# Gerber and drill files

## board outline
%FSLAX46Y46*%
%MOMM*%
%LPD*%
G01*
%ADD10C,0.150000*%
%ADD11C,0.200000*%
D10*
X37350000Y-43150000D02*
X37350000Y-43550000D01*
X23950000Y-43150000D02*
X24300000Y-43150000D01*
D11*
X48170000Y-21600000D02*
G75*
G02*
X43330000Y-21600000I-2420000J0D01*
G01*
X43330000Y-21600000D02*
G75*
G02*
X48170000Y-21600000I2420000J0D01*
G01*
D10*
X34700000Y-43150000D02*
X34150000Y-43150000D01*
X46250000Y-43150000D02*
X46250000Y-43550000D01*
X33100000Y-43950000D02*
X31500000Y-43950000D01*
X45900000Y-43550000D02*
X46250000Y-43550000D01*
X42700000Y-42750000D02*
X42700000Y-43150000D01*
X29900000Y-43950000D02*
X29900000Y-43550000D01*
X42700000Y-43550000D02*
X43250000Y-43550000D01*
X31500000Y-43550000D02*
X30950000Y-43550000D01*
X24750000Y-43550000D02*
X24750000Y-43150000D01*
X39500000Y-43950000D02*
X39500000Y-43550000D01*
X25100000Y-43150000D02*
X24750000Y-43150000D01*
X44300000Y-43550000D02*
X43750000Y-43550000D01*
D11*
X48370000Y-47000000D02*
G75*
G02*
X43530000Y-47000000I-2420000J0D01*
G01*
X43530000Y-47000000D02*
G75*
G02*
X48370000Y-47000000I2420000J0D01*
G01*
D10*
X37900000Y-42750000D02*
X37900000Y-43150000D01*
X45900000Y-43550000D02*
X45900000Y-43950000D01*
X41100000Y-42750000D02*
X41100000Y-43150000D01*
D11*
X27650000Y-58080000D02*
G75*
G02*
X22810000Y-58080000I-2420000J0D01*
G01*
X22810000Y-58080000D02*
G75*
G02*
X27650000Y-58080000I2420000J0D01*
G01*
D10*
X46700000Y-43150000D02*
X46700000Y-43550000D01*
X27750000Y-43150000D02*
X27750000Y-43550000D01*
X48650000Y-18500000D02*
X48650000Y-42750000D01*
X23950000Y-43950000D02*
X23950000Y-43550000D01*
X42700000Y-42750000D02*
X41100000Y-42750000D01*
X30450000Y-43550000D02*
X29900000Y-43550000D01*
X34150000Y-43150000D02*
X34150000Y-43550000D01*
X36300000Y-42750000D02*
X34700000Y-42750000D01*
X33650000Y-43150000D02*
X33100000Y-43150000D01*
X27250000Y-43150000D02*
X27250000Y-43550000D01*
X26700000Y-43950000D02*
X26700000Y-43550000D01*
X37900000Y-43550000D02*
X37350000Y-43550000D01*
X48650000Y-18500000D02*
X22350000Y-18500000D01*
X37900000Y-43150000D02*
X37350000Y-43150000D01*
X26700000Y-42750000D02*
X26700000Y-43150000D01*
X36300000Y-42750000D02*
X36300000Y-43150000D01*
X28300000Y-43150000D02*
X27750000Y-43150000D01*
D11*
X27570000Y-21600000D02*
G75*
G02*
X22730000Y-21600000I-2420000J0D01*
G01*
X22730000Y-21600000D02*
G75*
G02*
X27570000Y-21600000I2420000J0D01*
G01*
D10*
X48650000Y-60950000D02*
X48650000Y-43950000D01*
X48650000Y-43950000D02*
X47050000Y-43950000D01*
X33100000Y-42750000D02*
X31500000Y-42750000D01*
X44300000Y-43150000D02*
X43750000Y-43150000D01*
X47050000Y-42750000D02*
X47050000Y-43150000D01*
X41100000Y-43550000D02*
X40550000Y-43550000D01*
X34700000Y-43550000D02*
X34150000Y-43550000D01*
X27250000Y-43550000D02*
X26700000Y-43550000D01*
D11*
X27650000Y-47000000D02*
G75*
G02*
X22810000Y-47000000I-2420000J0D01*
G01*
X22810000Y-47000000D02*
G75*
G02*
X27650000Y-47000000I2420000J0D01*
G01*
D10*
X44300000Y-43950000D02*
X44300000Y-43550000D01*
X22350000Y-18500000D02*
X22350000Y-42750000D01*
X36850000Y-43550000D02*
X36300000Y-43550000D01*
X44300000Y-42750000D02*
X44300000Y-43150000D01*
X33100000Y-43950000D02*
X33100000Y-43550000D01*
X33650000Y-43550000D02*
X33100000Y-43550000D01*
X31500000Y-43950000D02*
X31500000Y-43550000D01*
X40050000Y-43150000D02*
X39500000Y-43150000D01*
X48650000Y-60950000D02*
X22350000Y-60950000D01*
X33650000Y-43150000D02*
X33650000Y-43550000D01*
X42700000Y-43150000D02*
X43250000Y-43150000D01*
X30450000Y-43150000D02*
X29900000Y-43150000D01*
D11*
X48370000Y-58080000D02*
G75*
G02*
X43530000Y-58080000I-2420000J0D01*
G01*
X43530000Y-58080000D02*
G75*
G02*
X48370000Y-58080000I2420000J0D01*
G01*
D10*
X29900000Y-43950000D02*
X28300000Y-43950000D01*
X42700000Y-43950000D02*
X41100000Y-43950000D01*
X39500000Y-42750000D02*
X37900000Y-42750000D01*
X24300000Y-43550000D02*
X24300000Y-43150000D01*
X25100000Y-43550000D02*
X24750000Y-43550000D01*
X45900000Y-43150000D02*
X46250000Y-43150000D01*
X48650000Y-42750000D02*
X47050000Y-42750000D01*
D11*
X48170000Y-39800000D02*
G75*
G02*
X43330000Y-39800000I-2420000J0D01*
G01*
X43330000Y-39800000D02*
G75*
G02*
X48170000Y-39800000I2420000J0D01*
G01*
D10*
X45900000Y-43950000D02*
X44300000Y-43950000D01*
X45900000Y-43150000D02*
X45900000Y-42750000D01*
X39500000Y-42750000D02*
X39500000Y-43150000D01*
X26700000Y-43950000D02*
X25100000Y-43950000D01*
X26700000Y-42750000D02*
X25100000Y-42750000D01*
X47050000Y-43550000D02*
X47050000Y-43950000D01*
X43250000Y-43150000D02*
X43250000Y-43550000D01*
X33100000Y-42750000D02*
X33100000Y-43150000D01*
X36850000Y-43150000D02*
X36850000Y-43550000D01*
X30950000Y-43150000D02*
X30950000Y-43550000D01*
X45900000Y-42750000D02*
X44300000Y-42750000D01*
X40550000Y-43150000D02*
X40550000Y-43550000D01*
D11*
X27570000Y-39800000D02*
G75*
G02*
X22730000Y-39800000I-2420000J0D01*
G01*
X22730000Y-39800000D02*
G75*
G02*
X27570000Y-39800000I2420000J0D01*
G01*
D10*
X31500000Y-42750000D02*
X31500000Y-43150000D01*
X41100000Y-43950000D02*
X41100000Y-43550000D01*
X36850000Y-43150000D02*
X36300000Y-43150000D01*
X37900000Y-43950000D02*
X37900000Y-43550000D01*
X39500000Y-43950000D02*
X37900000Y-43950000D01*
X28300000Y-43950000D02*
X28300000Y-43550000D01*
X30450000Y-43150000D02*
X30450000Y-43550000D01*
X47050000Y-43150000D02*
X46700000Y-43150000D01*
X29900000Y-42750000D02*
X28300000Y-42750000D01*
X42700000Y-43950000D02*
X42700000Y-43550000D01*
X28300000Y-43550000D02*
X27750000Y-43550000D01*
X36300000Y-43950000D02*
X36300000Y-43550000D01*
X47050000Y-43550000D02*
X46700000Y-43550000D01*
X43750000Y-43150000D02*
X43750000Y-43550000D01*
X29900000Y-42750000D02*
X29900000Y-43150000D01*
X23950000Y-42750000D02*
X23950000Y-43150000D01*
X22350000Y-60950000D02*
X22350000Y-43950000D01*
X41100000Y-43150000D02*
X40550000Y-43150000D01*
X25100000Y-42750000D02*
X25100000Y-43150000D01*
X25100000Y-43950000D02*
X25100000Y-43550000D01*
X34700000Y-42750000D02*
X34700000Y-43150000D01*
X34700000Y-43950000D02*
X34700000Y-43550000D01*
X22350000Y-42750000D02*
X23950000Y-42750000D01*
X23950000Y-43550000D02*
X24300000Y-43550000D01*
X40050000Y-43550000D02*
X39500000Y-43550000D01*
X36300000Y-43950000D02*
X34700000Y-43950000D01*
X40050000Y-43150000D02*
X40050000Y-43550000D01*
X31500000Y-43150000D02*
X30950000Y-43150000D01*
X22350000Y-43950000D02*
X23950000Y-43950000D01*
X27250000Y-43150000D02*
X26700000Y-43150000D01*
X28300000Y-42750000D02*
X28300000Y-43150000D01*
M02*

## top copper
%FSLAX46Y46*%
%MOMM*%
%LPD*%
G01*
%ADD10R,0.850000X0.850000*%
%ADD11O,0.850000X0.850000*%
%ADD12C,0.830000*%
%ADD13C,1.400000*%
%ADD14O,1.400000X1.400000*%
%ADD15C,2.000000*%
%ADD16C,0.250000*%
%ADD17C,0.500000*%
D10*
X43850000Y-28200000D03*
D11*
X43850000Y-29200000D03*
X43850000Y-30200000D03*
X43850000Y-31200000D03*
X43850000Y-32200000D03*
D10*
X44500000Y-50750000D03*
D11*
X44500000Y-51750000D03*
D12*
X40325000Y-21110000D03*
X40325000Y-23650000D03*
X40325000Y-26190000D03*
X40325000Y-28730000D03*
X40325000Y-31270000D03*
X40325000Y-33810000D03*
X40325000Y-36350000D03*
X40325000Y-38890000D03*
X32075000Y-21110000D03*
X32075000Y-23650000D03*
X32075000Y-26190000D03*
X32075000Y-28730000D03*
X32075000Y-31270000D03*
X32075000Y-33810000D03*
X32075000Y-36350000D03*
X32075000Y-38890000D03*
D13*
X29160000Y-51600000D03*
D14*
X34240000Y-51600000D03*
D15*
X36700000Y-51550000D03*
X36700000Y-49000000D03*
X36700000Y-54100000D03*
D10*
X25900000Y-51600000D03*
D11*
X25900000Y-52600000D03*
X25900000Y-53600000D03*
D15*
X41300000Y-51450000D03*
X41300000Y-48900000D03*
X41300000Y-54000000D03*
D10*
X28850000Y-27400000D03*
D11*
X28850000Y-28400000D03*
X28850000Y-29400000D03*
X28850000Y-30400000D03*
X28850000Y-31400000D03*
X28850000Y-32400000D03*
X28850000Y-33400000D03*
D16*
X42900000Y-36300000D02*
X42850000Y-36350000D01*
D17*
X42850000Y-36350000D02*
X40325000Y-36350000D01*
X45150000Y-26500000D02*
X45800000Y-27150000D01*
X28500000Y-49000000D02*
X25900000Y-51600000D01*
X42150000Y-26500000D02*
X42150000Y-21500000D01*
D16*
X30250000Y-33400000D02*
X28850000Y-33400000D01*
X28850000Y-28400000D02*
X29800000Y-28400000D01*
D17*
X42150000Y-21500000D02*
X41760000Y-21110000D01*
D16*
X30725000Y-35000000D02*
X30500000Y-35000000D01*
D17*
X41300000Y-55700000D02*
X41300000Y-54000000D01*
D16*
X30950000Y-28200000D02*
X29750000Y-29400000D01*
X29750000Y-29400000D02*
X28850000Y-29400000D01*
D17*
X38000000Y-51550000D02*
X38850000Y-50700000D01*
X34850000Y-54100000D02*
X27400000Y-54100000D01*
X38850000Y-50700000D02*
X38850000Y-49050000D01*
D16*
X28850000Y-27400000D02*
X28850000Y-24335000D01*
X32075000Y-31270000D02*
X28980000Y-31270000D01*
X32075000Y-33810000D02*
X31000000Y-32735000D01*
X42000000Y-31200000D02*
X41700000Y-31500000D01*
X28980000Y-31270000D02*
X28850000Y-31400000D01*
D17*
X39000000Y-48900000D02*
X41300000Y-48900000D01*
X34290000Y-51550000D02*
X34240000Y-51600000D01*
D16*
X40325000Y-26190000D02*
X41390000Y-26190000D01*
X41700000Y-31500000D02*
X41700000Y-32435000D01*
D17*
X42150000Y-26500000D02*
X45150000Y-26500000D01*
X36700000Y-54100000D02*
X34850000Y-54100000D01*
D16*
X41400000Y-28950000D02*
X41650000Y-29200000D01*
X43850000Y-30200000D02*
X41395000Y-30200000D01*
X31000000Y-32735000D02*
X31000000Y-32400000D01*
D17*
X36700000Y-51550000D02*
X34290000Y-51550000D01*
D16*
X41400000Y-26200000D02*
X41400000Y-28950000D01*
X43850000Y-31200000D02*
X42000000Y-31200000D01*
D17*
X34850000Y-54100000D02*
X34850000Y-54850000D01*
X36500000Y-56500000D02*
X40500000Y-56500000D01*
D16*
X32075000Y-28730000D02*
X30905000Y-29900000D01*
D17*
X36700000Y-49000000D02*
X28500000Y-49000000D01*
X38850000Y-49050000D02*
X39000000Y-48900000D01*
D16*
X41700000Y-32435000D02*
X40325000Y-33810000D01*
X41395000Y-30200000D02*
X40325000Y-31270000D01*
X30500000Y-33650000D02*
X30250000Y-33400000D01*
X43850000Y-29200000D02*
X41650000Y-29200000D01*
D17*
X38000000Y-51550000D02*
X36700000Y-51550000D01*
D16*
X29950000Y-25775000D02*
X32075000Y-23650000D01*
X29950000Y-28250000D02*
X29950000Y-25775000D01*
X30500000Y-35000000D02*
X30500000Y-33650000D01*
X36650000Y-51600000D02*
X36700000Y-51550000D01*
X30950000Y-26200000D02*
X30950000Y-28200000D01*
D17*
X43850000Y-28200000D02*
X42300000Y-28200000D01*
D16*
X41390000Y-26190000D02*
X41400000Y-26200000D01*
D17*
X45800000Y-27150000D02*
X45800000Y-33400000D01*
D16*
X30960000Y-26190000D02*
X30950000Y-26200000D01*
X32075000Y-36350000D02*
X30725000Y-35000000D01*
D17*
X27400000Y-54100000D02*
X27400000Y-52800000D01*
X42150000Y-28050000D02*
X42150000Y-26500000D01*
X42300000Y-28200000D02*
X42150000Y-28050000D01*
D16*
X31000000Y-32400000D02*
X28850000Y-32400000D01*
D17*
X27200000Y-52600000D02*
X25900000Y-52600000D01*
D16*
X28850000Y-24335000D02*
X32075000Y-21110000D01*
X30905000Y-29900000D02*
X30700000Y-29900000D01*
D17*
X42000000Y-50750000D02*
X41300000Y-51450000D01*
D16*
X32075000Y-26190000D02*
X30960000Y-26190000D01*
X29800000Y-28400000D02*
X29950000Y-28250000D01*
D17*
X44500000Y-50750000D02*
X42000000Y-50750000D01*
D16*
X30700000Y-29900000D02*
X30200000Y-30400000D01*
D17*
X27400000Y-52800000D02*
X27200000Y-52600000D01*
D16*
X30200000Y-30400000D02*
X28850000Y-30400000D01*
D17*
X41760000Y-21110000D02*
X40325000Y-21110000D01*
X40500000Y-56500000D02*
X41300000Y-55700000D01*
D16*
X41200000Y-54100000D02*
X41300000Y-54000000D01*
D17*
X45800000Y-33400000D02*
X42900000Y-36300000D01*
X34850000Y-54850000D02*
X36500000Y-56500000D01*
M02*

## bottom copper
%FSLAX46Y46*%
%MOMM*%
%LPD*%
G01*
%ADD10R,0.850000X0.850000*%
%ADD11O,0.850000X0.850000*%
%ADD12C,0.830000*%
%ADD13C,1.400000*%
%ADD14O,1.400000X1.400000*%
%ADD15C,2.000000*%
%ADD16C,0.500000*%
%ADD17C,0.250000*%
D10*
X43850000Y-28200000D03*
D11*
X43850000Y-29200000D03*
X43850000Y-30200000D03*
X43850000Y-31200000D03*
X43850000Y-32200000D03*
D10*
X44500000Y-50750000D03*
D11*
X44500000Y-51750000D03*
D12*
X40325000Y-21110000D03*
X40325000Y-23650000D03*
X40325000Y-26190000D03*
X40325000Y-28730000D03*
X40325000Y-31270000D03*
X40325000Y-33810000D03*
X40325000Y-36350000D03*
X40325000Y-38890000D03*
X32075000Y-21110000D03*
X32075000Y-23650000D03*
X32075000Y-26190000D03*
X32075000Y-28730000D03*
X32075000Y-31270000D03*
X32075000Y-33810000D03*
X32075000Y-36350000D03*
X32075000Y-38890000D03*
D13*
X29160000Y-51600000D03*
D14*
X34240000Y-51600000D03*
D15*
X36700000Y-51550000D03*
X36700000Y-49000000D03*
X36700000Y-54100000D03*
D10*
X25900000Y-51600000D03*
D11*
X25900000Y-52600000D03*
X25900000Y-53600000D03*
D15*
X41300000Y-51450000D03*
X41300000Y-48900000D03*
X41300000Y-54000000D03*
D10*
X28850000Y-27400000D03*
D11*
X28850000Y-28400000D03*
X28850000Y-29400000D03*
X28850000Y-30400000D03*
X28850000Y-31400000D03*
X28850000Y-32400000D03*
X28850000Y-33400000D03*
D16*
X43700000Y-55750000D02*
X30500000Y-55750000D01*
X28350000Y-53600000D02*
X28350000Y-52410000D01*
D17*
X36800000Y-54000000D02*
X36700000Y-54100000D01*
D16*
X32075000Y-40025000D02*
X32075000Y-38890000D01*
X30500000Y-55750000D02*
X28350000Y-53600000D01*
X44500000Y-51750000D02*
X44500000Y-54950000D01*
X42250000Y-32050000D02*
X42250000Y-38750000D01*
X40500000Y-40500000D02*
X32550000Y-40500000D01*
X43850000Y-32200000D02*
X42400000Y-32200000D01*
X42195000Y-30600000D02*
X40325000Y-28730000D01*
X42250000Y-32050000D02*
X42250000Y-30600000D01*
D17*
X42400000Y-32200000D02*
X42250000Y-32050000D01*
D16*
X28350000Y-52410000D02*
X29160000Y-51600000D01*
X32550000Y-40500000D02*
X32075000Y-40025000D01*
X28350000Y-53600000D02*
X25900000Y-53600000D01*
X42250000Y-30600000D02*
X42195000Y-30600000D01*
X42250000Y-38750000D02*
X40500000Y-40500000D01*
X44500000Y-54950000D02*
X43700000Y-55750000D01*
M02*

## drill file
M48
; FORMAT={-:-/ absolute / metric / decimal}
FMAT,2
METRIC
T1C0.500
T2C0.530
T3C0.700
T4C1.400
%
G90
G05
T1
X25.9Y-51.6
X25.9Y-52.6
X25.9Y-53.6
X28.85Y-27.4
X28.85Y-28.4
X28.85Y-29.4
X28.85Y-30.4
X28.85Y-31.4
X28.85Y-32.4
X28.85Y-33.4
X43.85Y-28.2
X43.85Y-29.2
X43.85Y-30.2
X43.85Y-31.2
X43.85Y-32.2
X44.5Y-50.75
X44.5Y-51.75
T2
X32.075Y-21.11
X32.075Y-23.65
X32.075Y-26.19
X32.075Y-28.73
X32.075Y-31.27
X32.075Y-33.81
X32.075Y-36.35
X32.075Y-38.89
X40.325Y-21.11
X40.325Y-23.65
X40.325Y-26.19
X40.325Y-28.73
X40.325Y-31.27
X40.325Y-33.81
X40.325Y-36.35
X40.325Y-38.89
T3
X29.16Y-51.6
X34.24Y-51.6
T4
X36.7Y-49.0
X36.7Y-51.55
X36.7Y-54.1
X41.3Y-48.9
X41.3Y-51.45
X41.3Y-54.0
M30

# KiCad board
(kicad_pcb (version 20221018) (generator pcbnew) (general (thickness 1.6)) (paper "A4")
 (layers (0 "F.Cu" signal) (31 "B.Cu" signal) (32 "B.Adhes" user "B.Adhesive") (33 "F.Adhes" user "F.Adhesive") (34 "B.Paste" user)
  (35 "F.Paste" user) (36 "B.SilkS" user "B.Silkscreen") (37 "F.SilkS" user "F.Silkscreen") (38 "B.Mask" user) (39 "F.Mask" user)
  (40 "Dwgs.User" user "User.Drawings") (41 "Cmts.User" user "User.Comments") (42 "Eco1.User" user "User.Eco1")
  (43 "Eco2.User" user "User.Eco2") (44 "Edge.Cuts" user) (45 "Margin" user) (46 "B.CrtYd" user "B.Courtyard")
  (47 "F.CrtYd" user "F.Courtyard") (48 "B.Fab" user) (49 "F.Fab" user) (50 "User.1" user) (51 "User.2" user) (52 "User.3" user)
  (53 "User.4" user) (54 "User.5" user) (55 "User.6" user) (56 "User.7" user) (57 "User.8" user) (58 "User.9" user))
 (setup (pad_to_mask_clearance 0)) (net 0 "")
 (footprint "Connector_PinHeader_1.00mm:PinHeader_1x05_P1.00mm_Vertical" (layer "F.Cu") (at 43.85 28.2)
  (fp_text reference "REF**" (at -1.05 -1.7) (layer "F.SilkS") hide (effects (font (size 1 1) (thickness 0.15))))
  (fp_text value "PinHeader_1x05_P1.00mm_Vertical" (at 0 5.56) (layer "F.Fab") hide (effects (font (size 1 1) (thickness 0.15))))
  (pad "1" thru_hole rect (at 0 0) (size 0.85 0.85) (drill 0.5) (layers "*.Cu" "*.Mask"))
  (pad "2" thru_hole oval (at 0 1) (size 0.85 0.85) (drill 0.5) (layers "*.Cu" "*.Mask"))
  (pad "3" thru_hole oval (at 0 2) (size 0.85 0.85) (drill 0.5) (layers "*.Cu" "*.Mask"))
  (pad "4" thru_hole oval (at 0 3) (size 0.85 0.85) (drill 0.5) (layers "*.Cu" "*.Mask"))
  (pad "5" thru_hole oval (at 0 4) (size 0.85 0.85) (drill 0.5) (layers "*.Cu" "*.Mask")))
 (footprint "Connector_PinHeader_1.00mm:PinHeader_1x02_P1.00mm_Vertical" (layer "F.Cu") (at 44.5 50.75)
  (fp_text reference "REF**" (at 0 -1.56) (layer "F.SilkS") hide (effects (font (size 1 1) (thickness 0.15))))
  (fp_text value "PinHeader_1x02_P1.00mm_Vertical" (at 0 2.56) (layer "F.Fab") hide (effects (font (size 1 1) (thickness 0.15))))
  (pad "1" thru_hole rect (at 0 0) (size 0.85 0.85) (drill 0.5) (layers "*.Cu" "*.Mask"))
  (pad "2" thru_hole oval (at 0 1) (size 0.85 0.85) (drill 0.5) (layers "*.Cu" "*.Mask")))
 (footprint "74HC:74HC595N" (layer "F.Cu") (at 36.2 30 -90)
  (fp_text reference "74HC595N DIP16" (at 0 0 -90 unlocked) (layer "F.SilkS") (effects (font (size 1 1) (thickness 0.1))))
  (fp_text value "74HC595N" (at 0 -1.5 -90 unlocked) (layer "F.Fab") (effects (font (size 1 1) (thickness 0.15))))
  (pad "1" thru_hole circle (at -8.89 -4.125 270) (size 0.83 0.83) (drill 0.53) (layers "*.Cu" "*.Mask"))
  (pad "2" thru_hole circle (at -6.35 -4.125 270) (size 0.83 0.83) (drill 0.53) (layers "*.Cu" "*.Mask"))
  (pad "3" thru_hole circle (at -3.81 -4.125 270) (size 0.83 0.83) (drill 0.53) (layers "*.Cu" "*.Mask"))
  (pad "4" thru_hole circle (at -1.27 -4.125 270) (size 0.83 0.83) (drill 0.53) (layers "*.Cu" "*.Mask"))
  (pad "5" thru_hole circle (at 1.27 -4.125 270) (size 0.83 0.83) (drill 0.53) (layers "*.Cu" "*.Mask"))
  (pad "6" thru_hole circle (at 3.81 -4.125 270) (size 0.83 0.83) (drill 0.53) (layers "*.Cu" "*.Mask"))
  (pad "7" thru_hole circle (at 6.35 -4.125 270) (size 0.83 0.83) (drill 0.53) (layers "*.Cu" "*.Mask"))
  (pad "8" thru_hole circle (at 8.89 -4.125 270) (size 0.83 0.83) (drill 0.53) (layers "*.Cu" "*.Mask"))
  (pad "9" thru_hole circle (at -8.89 4.125 270) (size 0.83 0.83) (drill 0.53) (layers "*.Cu" "*.Mask"))
  (pad "10" thru_hole circle (at -6.35 4.125 270) (size 0.83 0.83) (drill 0.53) (layers "*.Cu" "*.Mask"))
  (pad "11" thru_hole circle (at -3.81 4.125 270) (size 0.83 0.83) (drill 0.53) (layers "*.Cu" "*.Mask"))
  (pad "12" thru_hole circle (at -1.27 4.125 270) (size 0.83 0.83) (drill 0.53) (layers "*.Cu" "*.Mask"))
  (pad "13" thru_hole circle (at 1.27 4.125 270) (size 0.83 0.83) (drill 0.53) (layers "*.Cu" "*.Mask"))
  (pad "14" thru_hole circle (at 3.81 4.125 270) (size 0.83 0.83) (drill 0.53) (layers "*.Cu" "*.Mask"))
  (pad "15" thru_hole circle (at 6.35 4.125 270) (size 0.83 0.83) (drill 0.53) (layers "*.Cu" "*.Mask"))
  (pad "16" thru_hole circle (at 8.89 4.125 270) (size 0.83 0.83) (drill 0.53) (layers "*.Cu" "*.Mask")))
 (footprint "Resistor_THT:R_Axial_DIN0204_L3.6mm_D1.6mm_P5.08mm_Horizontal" (layer "F.Cu") (at 29.16 51.6)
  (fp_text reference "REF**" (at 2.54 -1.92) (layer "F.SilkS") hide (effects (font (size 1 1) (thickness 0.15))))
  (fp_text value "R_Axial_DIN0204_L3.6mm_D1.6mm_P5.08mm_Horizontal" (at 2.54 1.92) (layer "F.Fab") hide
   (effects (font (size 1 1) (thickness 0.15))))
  (pad "1" thru_hole circle (at 0 0) (size 1.4 1.4) (drill 0.7) (layers "*.Cu" "*.Mask"))
  (pad "2" thru_hole oval (at 5.08 0) (size 1.4 1.4) (drill 0.7) (layers "*.Cu" "*.Mask")))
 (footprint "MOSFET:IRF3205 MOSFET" (layer "F.Cu") (at 36.7 51.55)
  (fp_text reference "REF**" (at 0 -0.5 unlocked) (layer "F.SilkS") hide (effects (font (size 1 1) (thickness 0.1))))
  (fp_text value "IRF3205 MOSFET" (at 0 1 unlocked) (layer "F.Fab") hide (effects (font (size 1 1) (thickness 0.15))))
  (pad "D" thru_hole circle (at 0 0) (size 2 2) (drill 1.4) (layers "*.Cu" "*.Mask"))
  (pad "G" thru_hole circle (at 0 -2.55) (size 2 2) (drill 1.4) (layers "*.Cu" "*.Mask"))
  (pad "S" thru_hole circle (at 0 2.55) (size 2 2) (drill 1.4) (layers "*.Cu" "*.Mask")))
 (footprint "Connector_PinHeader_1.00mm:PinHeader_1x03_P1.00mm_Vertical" (layer "F.Cu") (at 25.9 51.6)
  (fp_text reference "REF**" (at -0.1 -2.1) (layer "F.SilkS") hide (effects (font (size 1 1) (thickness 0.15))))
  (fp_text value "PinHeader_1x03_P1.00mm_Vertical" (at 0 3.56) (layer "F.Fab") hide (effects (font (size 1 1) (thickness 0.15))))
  (pad "1" thru_hole rect (at 0 0) (size 0.85 0.85) (drill 0.5) (layers "*.Cu" "*.Mask"))
  (pad "2" thru_hole oval (at 0 1) (size 0.85 0.85) (drill 0.5) (layers "*.Cu" "*.Mask"))
  (pad "3" thru_hole oval (at 0 2) (size 0.85 0.85) (drill 0.5) (layers "*.Cu" "*.Mask")))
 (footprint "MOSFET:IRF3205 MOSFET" (layer "F.Cu") (at 41.3 51.45)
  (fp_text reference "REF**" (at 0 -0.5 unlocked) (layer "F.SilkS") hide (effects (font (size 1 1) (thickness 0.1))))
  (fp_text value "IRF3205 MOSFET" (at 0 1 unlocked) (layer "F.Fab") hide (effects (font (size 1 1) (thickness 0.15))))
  (pad "D" thru_hole circle (at 0 0) (size 2 2) (drill 1.4) (layers "*.Cu" "*.Mask"))
  (pad "G" thru_hole circle (at 0 -2.55) (size 2 2) (drill 1.4) (layers "*.Cu" "*.Mask"))
  (pad "S" thru_hole circle (at 0 2.55) (size 2 2) (drill 1.4) (layers "*.Cu" "*.Mask")))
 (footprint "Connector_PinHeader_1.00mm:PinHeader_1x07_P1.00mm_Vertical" (layer "F.Cu") (at 28.85 27.4)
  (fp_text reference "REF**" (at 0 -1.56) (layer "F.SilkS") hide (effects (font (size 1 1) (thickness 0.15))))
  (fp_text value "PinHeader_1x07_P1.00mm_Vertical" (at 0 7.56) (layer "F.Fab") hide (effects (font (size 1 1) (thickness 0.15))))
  (pad "1" thru_hole rect (at 0 0) (size 0.85 0.85) (drill 0.5) (layers "*.Cu" "*.Mask"))
  (pad "2" thru_hole oval (at 0 1) (size 0.85 0.85) (drill 0.5) (layers "*.Cu" "*.Mask"))
  (pad "3" thru_hole oval (at 0 2) (size 0.85 0.85) (drill 0.5) (layers "*.Cu" "*.Mask"))
  (pad "4" thru_hole oval (at 0 3) (size 0.85 0.85) (drill 0.5) (layers "*.Cu" "*.Mask"))
  (pad "5" thru_hole oval (at 0 4) (size 0.85 0.85) (drill 0.5) (layers "*.Cu" "*.Mask"))
  (pad "6" thru_hole oval (at 0 5) (size 0.85 0.85) (drill 0.5) (layers "*.Cu" "*.Mask"))
  (pad "7" thru_hole oval (at 0 6) (size 0.85 0.85) (drill 0.5) (layers "*.Cu" "*.Mask")))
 (gr_line (start 37.35 43.15) (end 37.35 43.55) (stroke (width 0.15) (type default)) (layer "Edge.Cuts"))
 (gr_line (start 23.95 43.15) (end 24.3 43.15) (stroke (width 0.15) (type default)) (layer "Edge.Cuts"))
 (gr_circle (center 45.75 21.6) (end 48.17 21.6) (stroke (width 0.2) (type default)) (fill none) (layer "Edge.Cuts"))
 (gr_line (start 34.7 43.15) (end 34.15 43.15) (stroke (width 0.15) (type default)) (layer "Edge.Cuts"))
 (gr_line (start 46.25 43.15) (end 46.25 43.55) (stroke (width 0.15) (type default)) (layer "Edge.Cuts"))
 (gr_line (start 33.1 43.95) (end 31.5 43.95) (stroke (width 0.15) (type default)) (layer "Edge.Cuts"))
 (gr_line (start 45.9 43.55) (end 46.25 43.55) (stroke (width 0.15) (type default)) (layer "Edge.Cuts"))
 (gr_line (start 42.7 42.75) (end 42.7 43.15) (stroke (width 0.15) (type default)) (layer "Edge.Cuts"))
 (gr_line (start 29.9 43.95) (end 29.9 43.55) (stroke (width 0.15) (type default)) (layer "Edge.Cuts"))
 (gr_line (start 42.7 43.55) (end 43.25 43.55) (stroke (width 0.15) (type default)) (layer "Edge.Cuts"))
 (gr_line (start 31.5 43.55) (end 30.95 43.55) (stroke (width 0.15) (type default)) (layer "Edge.Cuts"))
 (gr_line (start 24.75 43.55) (end 24.75 43.15) (stroke (width 0.15) (type default)) (layer "Edge.Cuts"))
 (gr_line (start 39.5 43.95) (end 39.5 43.55) (stroke (width 0.15) (type default)) (layer "Edge.Cuts"))
 (gr_line (start 25.1 43.15) (end 24.75 43.15) (stroke (width 0.15) (type default)) (layer "Edge.Cuts"))
 (gr_line (start 44.3 43.55) (end 43.75 43.55) (stroke (width 0.15) (type default)) (layer "Edge.Cuts"))
 (gr_circle (center 45.95 47) (end 48.37 47) (stroke (width 0.2) (type default)) (fill none) (layer "Edge.Cuts"))
 (gr_line (start 37.9 42.75) (end 37.9 43.15) (stroke (width 0.15) (type default)) (layer "Edge.Cuts"))
 (gr_line (start 45.9 43.55) (end 45.9 43.95) (stroke (width 0.15) (type default)) (layer "Edge.Cuts"))
 (gr_line (start 41.1 42.75) (end 41.1 43.15) (stroke (width 0.15) (type default)) (layer "Edge.Cuts"))
 (gr_circle (center 25.23 58.08) (end 27.65 58.08) (stroke (width 0.2) (type default)) (fill none) (layer "Edge.Cuts"))
 (gr_line (start 46.7 43.15) (end 46.7 43.55) (stroke (width 0.15) (type default)) (layer "Edge.Cuts"))
 (gr_line (start 27.75 43.15) (end 27.75 43.55) (stroke (width 0.15) (type default)) (layer "Edge.Cuts"))
 (gr_line (start 48.65 18.5) (end 48.65 42.75) (stroke (width 0.15) (type default)) (layer "Edge.Cuts"))
 (gr_line (start 23.95 43.95) (end 23.95 43.55) (stroke (width 0.15) (type default)) (layer "Edge.Cuts"))
 (gr_line (start 42.7 42.75) (end 41.1 42.75) (stroke (width 0.15) (type default)) (layer "Edge.Cuts"))
 (gr_line (start 30.45 43.55) (end 29.9 43.55) (stroke (width 0.15) (type default)) (layer "Edge.Cuts"))
 (gr_line (start 34.15 43.15) (end 34.15 43.55) (stroke (width 0.15) (type default)) (layer "Edge.Cuts"))
 (gr_line (start 36.3 42.75) (end 34.7 42.75) (stroke (width 0.15) (type default)) (layer "Edge.Cuts"))
 (gr_line (start 33.65 43.15) (end 33.1 43.15) (stroke (width 0.15) (type default)) (layer "Edge.Cuts"))
 (gr_line (start 27.25 43.15) (end 27.25 43.55) (stroke (width 0.15) (type default)) (layer "Edge.Cuts"))
 (gr_line (start 26.7 43.95) (end 26.7 43.55) (stroke (width 0.15) (type default)) (layer "Edge.Cuts"))
 (gr_line (start 37.9 43.55) (end 37.35 43.55) (stroke (width 0.15) (type default)) (layer "Edge.Cuts"))
 (gr_line (start 48.65 18.5) (end 22.35 18.5) (stroke (width 0.15) (type default)) (layer "Edge.Cuts"))
 (gr_line (start 37.9 43.15) (end 37.35 43.15) (stroke (width 0.15) (type default)) (layer "Edge.Cuts"))
 (gr_line (start 26.7 42.75) (end 26.7 43.15) (stroke (width 0.15) (type default)) (layer "Edge.Cuts"))
 (gr_line (start 36.3 42.75) (end 36.3 43.15) (stroke (width 0.15) (type default)) (layer "Edge.Cuts"))
 (gr_line (start 28.3 43.15) (end 27.75 43.15) (stroke (width 0.15) (type default)) (layer "Edge.Cuts"))
 (gr_circle (center 25.15 21.6) (end 27.57 21.6) (stroke (width 0.2) (type default)) (fill none) (layer "Edge.Cuts"))
 (gr_line (start 48.65 60.95) (end 48.65 43.95) (stroke (width 0.15) (type default)) (layer "Edge.Cuts"))
 (gr_line (start 48.65 43.95) (end 47.05 43.95) (stroke (width 0.15) (type default)) (layer "Edge.Cuts"))
 (gr_line (start 33.1 42.75) (end 31.5 42.75) (stroke (width 0.15) (type default)) (layer "Edge.Cuts"))
 (gr_line (start 44.3 43.15) (end 43.75 43.15) (stroke (width 0.15) (type default)) (layer "Edge.Cuts"))
 (gr_line (start 47.05 42.75) (end 47.05 43.15) (stroke (width 0.15) (type default)) (layer "Edge.Cuts"))
 (gr_line (start 41.1 43.55) (end 40.55 43.55) (stroke (width 0.15) (type default)) (layer "Edge.Cuts"))
 (gr_line (start 34.7 43.55) (end 34.15 43.55) (stroke (width 0.15) (type default)) (layer "Edge.Cuts"))
 (gr_line (start 27.25 43.55) (end 26.7 43.55) (stroke (width 0.15) (type default)) (layer "Edge.Cuts"))
 (gr_circle (center 25.23 47) (end 27.65 47) (stroke (width 0.2) (type default)) (fill none) (layer "Edge.Cuts"))
 (gr_line (start 44.3 43.95) (end 44.3 43.55) (stroke (width 0.15) (type default)) (layer "Edge.Cuts"))
 (gr_line (start 22.35 18.5) (end 22.35 42.75) (stroke (width 0.15) (type default)) (layer "Edge.Cuts"))
 (gr_line (start 36.85 43.55) (end 36.3 43.55) (stroke (width 0.15) (type default)) (layer "Edge.Cuts"))
 (gr_line (start 44.3 42.75) (end 44.3 43.15) (stroke (width 0.15) (type default)) (layer "Edge.Cuts"))
 (gr_line (start 33.1 43.95) (end 33.1 43.55) (stroke (width 0.15) (type default)) (layer "Edge.Cuts"))
 (gr_line (start 33.65 43.55) (end 33.1 43.55) (stroke (width 0.15) (type default)) (layer "Edge.Cuts"))
 (gr_line (start 31.5 43.95) (end 31.5 43.55) (stroke (width 0.15) (type default)) (layer "Edge.Cuts"))
 (gr_line (start 40.05 43.15) (end 39.5 43.15) (stroke (width 0.15) (type default)) (layer "Edge.Cuts"))
 (gr_line (start 48.65 60.95) (end 22.35 60.95) (stroke (width 0.15) (type default)) (layer "Edge.Cuts"))
 (gr_line (start 33.65 43.15) (end 33.65 43.55) (stroke (width 0.15) (type default)) (layer "Edge.Cuts"))
 (gr_line (start 42.7 43.15) (end 43.25 43.15) (stroke (width 0.15) (type default)) (layer "Edge.Cuts"))
 (gr_line (start 30.45 43.15) (end 29.9 43.15) (stroke (width 0.15) (type default)) (layer "Edge.Cuts"))
 (gr_circle (center 45.95 58.08) (end 48.37 58.08) (stroke (width 0.2) (type default)) (fill none) (layer "Edge.Cuts"))
 (gr_line (start 29.9 43.95) (end 28.3 43.95) (stroke (width 0.15) (type default)) (layer "Edge.Cuts"))
 (gr_line (start 42.7 43.95) (end 41.1 43.95) (stroke (width 0.15) (type default)) (layer "Edge.Cuts"))
 (gr_line (start 39.5 42.75) (end 37.9 42.75) (stroke (width 0.15) (type default)) (layer "Edge.Cuts"))
 (gr_line (start 24.3 43.55) (end 24.3 43.15) (stroke (width 0.15) (type default)) (layer "Edge.Cuts"))
 (gr_line (start 25.1 43.55) (end 24.75 43.55) (stroke (width 0.15) (type default)) (layer "Edge.Cuts"))
 (gr_line (start 45.9 43.15) (end 46.25 43.15) (stroke (width 0.15) (type default)) (layer "Edge.Cuts"))
 (gr_line (start 48.65 42.75) (end 47.05 42.75) (stroke (width 0.15) (type default)) (layer "Edge.Cuts"))
 (gr_circle (center 45.75 39.8) (end 48.17 39.8) (stroke (width 0.2) (type default)) (fill none) (layer "Edge.Cuts"))
 (gr_line (start 45.9 43.95) (end 44.3 43.95) (stroke (width 0.15) (type default)) (layer "Edge.Cuts"))
 (gr_line (start 45.9 43.15) (end 45.9 42.75) (stroke (width 0.15) (type default)) (layer "Edge.Cuts"))
 (gr_line (start 39.5 42.75) (end 39.5 43.15) (stroke (width 0.15) (type default)) (layer "Edge.Cuts"))
 (gr_line (start 26.7 43.95) (end 25.1 43.95) (stroke (width 0.15) (type default)) (layer "Edge.Cuts"))
 (gr_line (start 26.7 42.75) (end 25.1 42.75) (stroke (width 0.15) (type default)) (layer "Edge.Cuts"))
 (gr_line (start 47.05 43.55) (end 47.05 43.95) (stroke (width 0.15) (type default)) (layer "Edge.Cuts"))
 (gr_line (start 43.25 43.15) (end 43.25 43.55) (stroke (width 0.15) (type default)) (layer "Edge.Cuts"))
 (gr_line (start 33.1 42.75) (end 33.1 43.15) (stroke (width 0.15) (type default)) (layer "Edge.Cuts"))
 (gr_line (start 36.85 43.15) (end 36.85 43.55) (stroke (width 0.15) (type default)) (layer "Edge.Cuts"))
 (gr_line (start 30.95 43.15) (end 30.95 43.55) (stroke (width 0.15) (type default)) (layer "Edge.Cuts"))
 (gr_line (start 45.9 42.75) (end 44.3 42.75) (stroke (width 0.15) (type default)) (layer "Edge.Cuts"))
 (gr_line (start 40.55 43.15) (end 40.55 43.55) (stroke (width 0.15) (type default)) (layer "Edge.Cuts"))
 (gr_circle (center 25.15 39.8) (end 27.57 39.8) (stroke (width 0.2) (type default)) (fill none) (layer "Edge.Cuts"))
 (gr_line (start 31.5 42.75) (end 31.5 43.15) (stroke (width 0.15) (type default)) (layer "Edge.Cuts"))
 (gr_line (start 41.1 43.95) (end 41.1 43.55) (stroke (width 0.15) (type default)) (layer "Edge.Cuts"))
 (gr_line (start 36.85 43.15) (end 36.3 43.15) (stroke (width 0.15) (type default)) (layer "Edge.Cuts"))
 (gr_line (start 37.9 43.95) (end 37.9 43.55) (stroke (width 0.15) (type default)) (layer "Edge.Cuts"))
 (gr_line (start 39.5 43.95) (end 37.9 43.95) (stroke (width 0.15) (type default)) (layer "Edge.Cuts"))
 (gr_line (start 28.3 43.95) (end 28.3 43.55) (stroke (width 0.15) (type default)) (layer "Edge.Cuts"))
 (gr_line (start 30.45 43.15) (end 30.45 43.55) (stroke (width 0.15) (type default)) (layer "Edge.Cuts"))
 (gr_line (start 47.05 43.15) (end 46.7 43.15) (stroke (width 0.15) (type default)) (layer "Edge.Cuts"))
 (gr_line (start 29.9 42.75) (end 28.3 42.75) (stroke (width 0.15) (type default)) (layer "Edge.Cuts"))
 (gr_line (start 42.7 43.95) (end 42.7 43.55) (stroke (width 0.15) (type default)) (layer "Edge.Cuts"))
 (gr_line (start 28.3 43.55) (end 27.75 43.55) (stroke (width 0.15) (type default)) (layer "Edge.Cuts"))
 (gr_line (start 36.3 43.95) (end 36.3 43.55) (stroke (width 0.15) (type default)) (layer "Edge.Cuts"))
 (gr_line (start 47.05 43.55) (end 46.7 43.55) (stroke (width 0.15) (type default)) (layer "Edge.Cuts"))
 (gr_line (start 43.75 43.15) (end 43.75 43.55) (stroke (width 0.15) (type default)) (layer "Edge.Cuts"))
 (gr_line (start 29.9 42.75) (end 29.9 43.15) (stroke (width 0.15) (type default)) (layer "Edge.Cuts"))
 (gr_line (start 23.95 42.75) (end 23.95 43.15) (stroke (width 0.15) (type default)) (layer "Edge.Cuts"))
 (gr_line (start 22.35 60.95) (end 22.35 43.95) (stroke (width 0.15) (type default)) (layer "Edge.Cuts"))
 (gr_line (start 41.1 43.15) (end 40.55 43.15) (stroke (width 0.15) (type default)) (layer "Edge.Cuts"))
 (gr_line (start 25.1 42.75) (end 25.1 43.15) (stroke (width 0.15) (type default)) (layer "Edge.Cuts"))
 (gr_line (start 25.1 43.95) (end 25.1 43.55) (stroke (width 0.15) (type default)) (layer "Edge.Cuts"))
 (gr_line (start 34.7 42.75) (end 34.7 43.15) (stroke (width 0.15) (type default)) (layer "Edge.Cuts"))
 (gr_line (start 34.7 43.95) (end 34.7 43.55) (stroke (width 0.15) (type default)) (layer "Edge.Cuts"))
 (gr_line (start 22.35 42.75) (end 23.95 42.75) (stroke (width 0.15) (type default)) (layer "Edge.Cuts"))
 (gr_line (start 23.95 43.55) (end 24.3 43.55) (stroke (width 0.15) (type default)) (layer "Edge.Cuts"))
 (gr_line (start 40.05 43.55) (end 39.5 43.55) (stroke (width 0.15) (type default)) (layer "Edge.Cuts"))
 (gr_line (start 36.3 43.95) (end 34.7 43.95) (stroke (width 0.15) (type default)) (layer "Edge.Cuts"))
 (gr_line (start 40.05 43.15) (end 40.05 43.55) (stroke (width 0.15) (type default)) (layer "Edge.Cuts"))
 (gr_line (start 31.5 43.15) (end 30.95 43.15) (stroke (width 0.15) (type default)) (layer "Edge.Cuts"))
 (gr_line (start 22.35 43.95) (end 23.95 43.95) (stroke (width 0.15) (type default)) (layer "Edge.Cuts"))
 (gr_line (start 27.25 43.15) (end 26.7 43.15) (stroke (width 0.15) (type default)) (layer "Edge.Cuts"))
 (gr_line (start 28.3 42.75) (end 28.3 43.15) (stroke (width 0.15) (type default)) (layer "Edge.Cuts"))
 (segment (start 42.9 36.3) (end 42.85 36.35) (width 0.25) (layer "F.Cu") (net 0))
 (segment (start 42.85 36.35) (end 40.325 36.35) (width 0.5) (layer "F.Cu") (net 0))
 (segment (start 45.15 26.5) (end 45.8 27.15) (width 0.5) (layer "F.Cu") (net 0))
 (segment (start 28.5 49) (end 25.9 51.6) (width 0.5) (layer "F.Cu") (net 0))
 (segment (start 42.15 26.5) (end 42.15 21.5) (width 0.5) (layer "F.Cu") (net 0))
 (segment (start 30.25 33.4) (end 28.85 33.4) (width 0.25) (layer "F.Cu") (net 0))
 (segment (start 28.85 28.4) (end 29.8 28.4) (width 0.25) (layer "F.Cu") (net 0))
 (segment (start 42.15 21.5) (end 41.76 21.11) (width 0.5) (layer "F.Cu") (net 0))
 (segment (start 30.725 35) (end 30.5 35) (width 0.25) (layer "F.Cu") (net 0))
 (segment (start 41.3 55.7) (end 41.3 54) (width 0.5) (layer "F.Cu") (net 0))
 (segment (start 30.95 28.2) (end 29.75 29.4) (width 0.25) (layer "F.Cu") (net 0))
 (segment (start 29.75 29.4) (end 28.85 29.4) (width 0.25) (layer "F.Cu") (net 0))
 (segment (start 38 51.55) (end 38.85 50.7) (width 0.5) (layer "F.Cu") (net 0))
 (segment (start 34.85 54.1) (end 27.4 54.1) (width 0.5) (layer "F.Cu") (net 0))
 (segment (start 38.85 50.7) (end 38.85 49.05) (width 0.5) (layer "F.Cu") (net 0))
 (segment (start 28.85 27.4) (end 28.85 24.335) (width 0.25) (layer "F.Cu") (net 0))
 (segment (start 32.075 31.27) (end 28.98 31.27) (width 0.25) (layer "F.Cu") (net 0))
 (segment (start 32.075 33.81) (end 31 32.735) (width 0.25) (layer "F.Cu") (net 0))
 (segment (start 42 31.2) (end 41.7 31.5) (width 0.25) (layer "F.Cu") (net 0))
 (segment (start 28.98 31.27) (end 28.85 31.4) (width 0.25) (layer "F.Cu") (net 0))
 (segment (start 39 48.9) (end 41.3 48.9) (width 0.5) (layer "F.Cu") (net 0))
 (segment (start 34.29 51.55) (end 34.24 51.6) (width 0.5) (layer "F.Cu") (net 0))
 (segment (start 40.325 26.19) (end 41.39 26.19) (width 0.25) (layer "F.Cu") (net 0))
 (segment (start 41.7 31.5) (end 41.7 32.435) (width 0.25) (layer "F.Cu") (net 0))
 (segment (start 42.15 26.5) (end 45.15 26.5) (width 0.5) (layer "F.Cu") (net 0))
 (segment (start 36.7 54.1) (end 34.85 54.1) (width 0.5) (layer "F.Cu") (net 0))
 (segment (start 41.4 28.95) (end 41.65 29.2) (width 0.25) (layer "F.Cu") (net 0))
 (segment (start 43.85 30.2) (end 41.395 30.2) (width 0.25) (layer "F.Cu") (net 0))
 (segment (start 31 32.735) (end 31 32.4) (width 0.25) (layer "F.Cu") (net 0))
 (segment (start 36.7 51.55) (end 34.29 51.55) (width 0.5) (layer "F.Cu") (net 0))
 (segment (start 41.4 26.2) (end 41.4 28.95) (width 0.25) (layer "F.Cu") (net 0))
 (segment (start 43.85 31.2) (end 42 31.2) (width 0.25) (layer "F.Cu") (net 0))
 (segment (start 34.85 54.1) (end 34.85 54.85) (width 0.5) (layer "F.Cu") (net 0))
 (segment (start 36.5 56.5) (end 40.5 56.5) (width 0.5) (layer "F.Cu") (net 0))
 (segment (start 32.075 28.73) (end 30.905 29.9) (width 0.25) (layer "F.Cu") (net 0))
 (segment (start 36.7 49) (end 28.5 49) (width 0.5) (layer "F.Cu") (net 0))
 (segment (start 38.85 49.05) (end 39 48.9) (width 0.5) (layer "F.Cu") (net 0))
 (segment (start 41.7 32.435) (end 40.325 33.81) (width 0.25) (layer "F.Cu") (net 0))
 (segment (start 41.395 30.2) (end 40.325 31.27) (width 0.25) (layer "F.Cu") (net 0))
 (segment (start 30.5 33.65) (end 30.25 33.4) (width 0.25) (layer "F.Cu") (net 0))
 (segment (start 43.85 29.2) (end 41.65 29.2) (width 0.25) (layer "F.Cu") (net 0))
 (segment (start 38 51.55) (end 36.7 51.55) (width 0.5) (layer "F.Cu") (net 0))
 (segment (start 29.95 25.775) (end 32.075 23.65) (width 0.25) (layer "F.Cu") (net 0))
 (segment (start 29.95 28.25) (end 29.95 25.775) (width 0.25) (layer "F.Cu") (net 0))
 (segment (start 30.5 35) (end 30.5 33.65) (width 0.25) (layer "F.Cu") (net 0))
 (segment (start 36.65 51.6) (end 36.7 51.55) (width 0.25) (layer "F.Cu") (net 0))
 (segment (start 30.95 26.2) (end 30.95 28.2) (width 0.25) (layer "F.Cu") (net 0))
 (segment (start 43.85 28.2) (end 42.3 28.2) (width 0.5) (layer "F.Cu") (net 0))
 (segment (start 41.39 26.19) (end 41.4 26.2) (width 0.25) (layer "F.Cu") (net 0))
 (segment (start 45.8 27.15) (end 45.8 33.4) (width 0.5) (layer "F.Cu") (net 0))
 (segment (start 30.96 26.19) (end 30.95 26.2) (width 0.25) (layer "F.Cu") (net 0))
 (segment (start 32.075 36.35) (end 30.725 35) (width 0.25) (layer "F.Cu") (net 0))
 (segment (start 27.4 54.1) (end 27.4 52.8) (width 0.5) (layer "F.Cu") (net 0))
 (segment (start 42.15 28.05) (end 42.15 26.5) (width 0.5) (layer "F.Cu") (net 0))
 (segment (start 42.3 28.2) (end 42.15 28.05) (width 0.5) (layer "F.Cu") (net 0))
 (segment (start 31 32.4) (end 28.85 32.4) (width 0.25) (layer "F.Cu") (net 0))
 (segment (start 27.2 52.6) (end 25.9 52.6) (width 0.5) (layer "F.Cu") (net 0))
 (segment (start 28.85 24.335) (end 32.075 21.11) (width 0.25) (layer "F.Cu") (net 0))
 (segment (start 30.905 29.9) (end 30.7 29.9) (width 0.25) (layer "F.Cu") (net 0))
 (segment (start 42 50.75) (end 41.3 51.45) (width 0.5) (layer "F.Cu") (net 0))
 (segment (start 32.075 26.19) (end 30.96 26.19) (width 0.25) (layer "F.Cu") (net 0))
 (segment (start 29.8 28.4) (end 29.95 28.25) (width 0.25) (layer "F.Cu") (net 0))
 (segment (start 44.5 50.75) (end 42 50.75) (width 0.5) (layer "F.Cu") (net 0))
 (segment (start 30.7 29.9) (end 30.2 30.4) (width 0.25) (layer "F.Cu") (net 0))
 (segment (start 27.4 52.8) (end 27.2 52.6) (width 0.5) (layer "F.Cu") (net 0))
 (segment (start 30.2 30.4) (end 28.85 30.4) (width 0.25) (layer "F.Cu") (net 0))
 (segment (start 41.76 21.11) (end 40.325 21.11) (width 0.5) (layer "F.Cu") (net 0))
 (segment (start 40.5 56.5) (end 41.3 55.7) (width 0.5) (layer "F.Cu") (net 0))
 (segment (start 41.2 54.1) (end 41.3 54) (width 0.25) (layer "F.Cu") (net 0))
 (segment (start 45.8 33.4) (end 42.9 36.3) (width 0.5) (layer "F.Cu") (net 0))
 (segment (start 34.85 54.85) (end 36.5 56.5) (width 0.5) (layer "F.Cu") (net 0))
 (segment (start 43.7 55.75) (end 30.5 55.75) (width 0.5) (layer "B.Cu") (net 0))
 (segment (start 28.35 53.6) (end 28.35 52.41) (width 0.5) (layer "B.Cu") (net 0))
 (segment (start 36.8 54) (end 36.7 54.1) (width 0.25) (layer "B.Cu") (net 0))
 (segment (start 32.075 40.025) (end 32.075 38.89) (width 0.5) (layer "B.Cu") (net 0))
 (segment (start 30.5 55.75) (end 28.35 53.6) (width 0.5) (layer "B.Cu") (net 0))
 (segment (start 44.5 51.75) (end 44.5 54.95) (width 0.5) (layer "B.Cu") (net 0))
 (segment (start 42.25 32.05) (end 42.25 38.75) (width 0.5) (layer "B.Cu") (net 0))
 (segment (start 40.5 40.5) (end 32.55 40.5) (width 0.5) (layer "B.Cu") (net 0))
 (segment (start 43.85 32.2) (end 42.4 32.2) (width 0.5) (layer "B.Cu") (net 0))
 (segment (start 42.195 30.6) (end 40.325 28.73) (width 0.5) (layer "B.Cu") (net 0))
 (segment (start 42.25 32.05) (end 42.25 30.6) (width 0.5) (layer "B.Cu") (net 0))
 (segment (start 42.4 32.2) (end 42.25 32.05) (width 0.25) (layer "B.Cu") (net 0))
 (segment (start 28.35 52.41) (end 29.16 51.6) (width 0.5) (layer "B.Cu") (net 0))
 (segment (start 32.55 40.5) (end 32.075 40.025) (width 0.5) (layer "B.Cu") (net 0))
 (segment (start 28.35 53.6) (end 25.9 53.6) (width 0.5) (layer "B.Cu") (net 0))
 (segment (start 42.25 30.6) (end 42.195 30.6) (width 0.5) (layer "B.Cu") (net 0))
 (segment (start 42.25 38.75) (end 40.5 40.5) (width 0.5) (layer "B.Cu") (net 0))
 (segment (start 44.5 54.95) (end 43.7 55.75) (width 0.5) (layer "B.Cu") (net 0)))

